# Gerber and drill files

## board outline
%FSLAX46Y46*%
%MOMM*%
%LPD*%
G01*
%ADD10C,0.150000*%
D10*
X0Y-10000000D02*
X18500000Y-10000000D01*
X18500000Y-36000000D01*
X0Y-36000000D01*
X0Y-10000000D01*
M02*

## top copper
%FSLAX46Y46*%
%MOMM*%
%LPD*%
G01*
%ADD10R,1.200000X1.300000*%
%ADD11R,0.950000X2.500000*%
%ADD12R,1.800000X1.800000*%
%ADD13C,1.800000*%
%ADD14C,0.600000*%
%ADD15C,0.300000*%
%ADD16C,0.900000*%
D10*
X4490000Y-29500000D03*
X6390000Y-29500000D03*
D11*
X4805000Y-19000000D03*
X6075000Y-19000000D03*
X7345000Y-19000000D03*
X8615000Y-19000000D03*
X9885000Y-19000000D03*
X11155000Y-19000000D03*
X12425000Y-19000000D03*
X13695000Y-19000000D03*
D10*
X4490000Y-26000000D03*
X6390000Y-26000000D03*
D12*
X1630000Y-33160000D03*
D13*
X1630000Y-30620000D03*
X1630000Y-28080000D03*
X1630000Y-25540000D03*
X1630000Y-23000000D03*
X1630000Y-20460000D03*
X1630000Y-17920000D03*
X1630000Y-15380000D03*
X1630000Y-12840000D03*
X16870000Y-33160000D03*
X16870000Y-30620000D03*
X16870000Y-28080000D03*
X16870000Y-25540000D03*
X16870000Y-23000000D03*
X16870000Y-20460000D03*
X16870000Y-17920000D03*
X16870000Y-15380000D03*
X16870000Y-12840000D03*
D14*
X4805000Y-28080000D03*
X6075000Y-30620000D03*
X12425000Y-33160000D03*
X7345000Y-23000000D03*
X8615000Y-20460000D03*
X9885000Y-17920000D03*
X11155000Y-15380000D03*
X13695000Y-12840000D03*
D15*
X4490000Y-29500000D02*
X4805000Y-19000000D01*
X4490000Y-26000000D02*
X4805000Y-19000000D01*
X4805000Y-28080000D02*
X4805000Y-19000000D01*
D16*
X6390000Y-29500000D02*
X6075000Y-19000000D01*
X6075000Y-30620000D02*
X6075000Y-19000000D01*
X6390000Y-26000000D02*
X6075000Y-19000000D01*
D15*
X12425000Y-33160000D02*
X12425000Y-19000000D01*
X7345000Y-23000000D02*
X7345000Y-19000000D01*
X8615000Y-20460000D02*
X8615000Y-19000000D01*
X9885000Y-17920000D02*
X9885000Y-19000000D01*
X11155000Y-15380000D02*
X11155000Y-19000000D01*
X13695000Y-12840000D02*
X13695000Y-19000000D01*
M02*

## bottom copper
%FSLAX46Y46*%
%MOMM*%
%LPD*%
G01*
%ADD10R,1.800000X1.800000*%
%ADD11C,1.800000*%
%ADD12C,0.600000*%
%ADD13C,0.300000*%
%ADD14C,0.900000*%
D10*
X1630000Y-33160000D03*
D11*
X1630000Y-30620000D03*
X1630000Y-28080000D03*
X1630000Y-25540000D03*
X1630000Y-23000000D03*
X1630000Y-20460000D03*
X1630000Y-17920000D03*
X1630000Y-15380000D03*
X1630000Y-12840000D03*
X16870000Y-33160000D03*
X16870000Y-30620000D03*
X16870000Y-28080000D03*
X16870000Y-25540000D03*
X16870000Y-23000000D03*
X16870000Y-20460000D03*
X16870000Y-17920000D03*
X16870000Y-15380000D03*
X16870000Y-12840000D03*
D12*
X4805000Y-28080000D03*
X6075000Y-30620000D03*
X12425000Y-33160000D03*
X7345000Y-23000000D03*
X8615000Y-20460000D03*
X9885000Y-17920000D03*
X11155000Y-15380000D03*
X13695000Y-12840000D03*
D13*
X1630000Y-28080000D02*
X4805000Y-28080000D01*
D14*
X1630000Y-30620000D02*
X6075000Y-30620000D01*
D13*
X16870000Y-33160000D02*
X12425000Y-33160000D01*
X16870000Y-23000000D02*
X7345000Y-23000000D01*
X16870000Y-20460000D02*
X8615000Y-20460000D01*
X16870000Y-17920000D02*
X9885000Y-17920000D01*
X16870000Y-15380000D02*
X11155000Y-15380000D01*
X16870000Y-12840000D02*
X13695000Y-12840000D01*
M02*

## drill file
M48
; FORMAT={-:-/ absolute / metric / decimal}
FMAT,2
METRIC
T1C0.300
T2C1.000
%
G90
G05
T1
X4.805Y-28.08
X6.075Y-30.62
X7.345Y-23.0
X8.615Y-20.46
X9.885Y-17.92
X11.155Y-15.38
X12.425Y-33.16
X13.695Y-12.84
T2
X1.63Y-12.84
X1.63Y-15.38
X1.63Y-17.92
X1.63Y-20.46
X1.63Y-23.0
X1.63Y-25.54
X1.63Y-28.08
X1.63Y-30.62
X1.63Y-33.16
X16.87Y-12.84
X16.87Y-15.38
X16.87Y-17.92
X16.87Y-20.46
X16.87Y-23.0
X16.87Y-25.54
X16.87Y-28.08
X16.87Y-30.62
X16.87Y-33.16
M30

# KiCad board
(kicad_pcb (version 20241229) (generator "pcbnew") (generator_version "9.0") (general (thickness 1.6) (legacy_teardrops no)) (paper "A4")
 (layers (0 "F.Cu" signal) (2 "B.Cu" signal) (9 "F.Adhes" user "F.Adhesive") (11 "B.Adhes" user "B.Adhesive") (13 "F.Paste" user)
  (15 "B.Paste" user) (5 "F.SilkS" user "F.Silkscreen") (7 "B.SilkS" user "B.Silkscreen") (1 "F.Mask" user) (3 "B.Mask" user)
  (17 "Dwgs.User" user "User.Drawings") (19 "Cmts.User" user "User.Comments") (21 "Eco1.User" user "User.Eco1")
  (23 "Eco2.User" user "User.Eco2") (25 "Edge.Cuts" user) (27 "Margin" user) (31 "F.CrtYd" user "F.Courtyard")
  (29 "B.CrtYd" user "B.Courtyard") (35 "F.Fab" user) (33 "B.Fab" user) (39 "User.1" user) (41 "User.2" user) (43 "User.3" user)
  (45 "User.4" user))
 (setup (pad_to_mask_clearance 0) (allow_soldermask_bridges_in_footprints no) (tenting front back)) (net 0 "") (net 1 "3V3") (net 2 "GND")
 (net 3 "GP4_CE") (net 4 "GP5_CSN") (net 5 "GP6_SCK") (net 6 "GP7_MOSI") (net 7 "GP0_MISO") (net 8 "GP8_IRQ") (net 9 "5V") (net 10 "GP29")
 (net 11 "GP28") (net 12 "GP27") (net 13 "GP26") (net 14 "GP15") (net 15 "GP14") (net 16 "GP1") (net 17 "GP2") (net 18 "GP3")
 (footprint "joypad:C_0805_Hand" (layer "F.Cu") (at 5.44 29.5)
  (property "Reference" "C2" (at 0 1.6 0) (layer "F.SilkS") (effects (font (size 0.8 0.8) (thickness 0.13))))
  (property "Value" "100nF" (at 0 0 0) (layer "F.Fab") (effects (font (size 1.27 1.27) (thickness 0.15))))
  (pad "1" smd rect (at -0.95 0) (size 1.2 1.3) (layers "F.Cu" "F.Mask" "F.Paste") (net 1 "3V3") (thermal_bridge_angle 45))
  (pad "2" smd rect (at 0.95 0) (size 1.2 1.3) (layers "F.Cu" "F.Mask" "F.Paste") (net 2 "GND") (thermal_bridge_angle 45)))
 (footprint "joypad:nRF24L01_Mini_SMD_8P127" (layer "F.Cu") (at 9.25 19)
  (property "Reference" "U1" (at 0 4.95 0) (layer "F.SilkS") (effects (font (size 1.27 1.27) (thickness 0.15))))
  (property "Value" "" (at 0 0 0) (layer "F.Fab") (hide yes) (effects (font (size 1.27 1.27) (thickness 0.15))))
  (pad "1" smd rect (at -4.445 0) (size 0.95 2.5) (layers "F.Cu" "F.Mask" "F.Paste") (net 1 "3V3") (thermal_bridge_angle 45))
  (pad "2" smd rect (at -3.175 0) (size 0.95 2.5) (layers "F.Cu" "F.Mask" "F.Paste") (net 2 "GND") (thermal_bridge_angle 45))
  (pad "3" smd rect (at -1.905 0) (size 0.95 2.5) (layers "F.Cu" "F.Mask" "F.Paste") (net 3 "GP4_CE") (thermal_bridge_angle 45))
  (pad "4" smd rect (at -0.635 0) (size 0.95 2.5) (layers "F.Cu" "F.Mask" "F.Paste") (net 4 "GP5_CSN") (thermal_bridge_angle 45))
  (pad "5" smd rect (at 0.635 0) (size 0.95 2.5) (layers "F.Cu" "F.Mask" "F.Paste") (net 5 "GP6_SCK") (thermal_bridge_angle 45))
  (pad "6" smd rect (at 1.905 0) (size 0.95 2.5) (layers "F.Cu" "F.Mask" "F.Paste") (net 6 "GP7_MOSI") (thermal_bridge_angle 45))
  (pad "7" smd rect (at 3.175 0) (size 0.95 2.5) (layers "F.Cu" "F.Mask" "F.Paste") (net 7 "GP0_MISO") (thermal_bridge_angle 45))
  (pad "8" smd rect (at 4.445 0) (size 0.95 2.5) (layers "F.Cu" "F.Mask" "F.Paste") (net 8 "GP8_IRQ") (thermal_bridge_angle 45))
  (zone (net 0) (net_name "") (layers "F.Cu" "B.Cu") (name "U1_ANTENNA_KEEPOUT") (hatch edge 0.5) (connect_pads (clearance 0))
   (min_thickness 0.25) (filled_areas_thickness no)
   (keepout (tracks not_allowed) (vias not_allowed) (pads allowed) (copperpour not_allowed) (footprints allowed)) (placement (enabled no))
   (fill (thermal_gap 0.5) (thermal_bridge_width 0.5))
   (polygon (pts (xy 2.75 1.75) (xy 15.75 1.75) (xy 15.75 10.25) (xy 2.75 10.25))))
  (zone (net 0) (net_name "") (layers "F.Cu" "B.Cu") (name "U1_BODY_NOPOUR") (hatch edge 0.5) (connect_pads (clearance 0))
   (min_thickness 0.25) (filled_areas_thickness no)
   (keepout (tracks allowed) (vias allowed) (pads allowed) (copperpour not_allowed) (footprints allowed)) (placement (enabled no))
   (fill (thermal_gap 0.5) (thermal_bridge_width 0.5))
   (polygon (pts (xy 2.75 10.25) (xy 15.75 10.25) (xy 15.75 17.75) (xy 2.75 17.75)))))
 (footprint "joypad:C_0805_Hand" (layer "F.Cu") (at 5.44 26)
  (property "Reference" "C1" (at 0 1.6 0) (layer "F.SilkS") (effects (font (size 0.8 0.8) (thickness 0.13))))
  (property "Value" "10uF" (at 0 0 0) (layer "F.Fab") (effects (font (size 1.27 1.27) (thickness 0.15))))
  (pad "1" smd rect (at -0.95 0) (size 1.2 1.3) (layers "F.Cu" "F.Mask" "F.Paste") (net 1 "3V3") (thermal_bridge_angle 45))
  (pad "2" smd rect (at 0.95 0) (size 1.2 1.3) (layers "F.Cu" "F.Mask" "F.Paste") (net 2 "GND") (thermal_bridge_angle 45)))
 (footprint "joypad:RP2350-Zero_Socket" (layer "F.Cu") (at 9.25 23)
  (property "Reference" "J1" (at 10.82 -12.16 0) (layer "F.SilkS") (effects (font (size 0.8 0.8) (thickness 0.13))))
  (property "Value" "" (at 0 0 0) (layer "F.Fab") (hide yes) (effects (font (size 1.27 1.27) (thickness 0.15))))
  (pad "1" thru_hole rect (at -7.62 10.16) (size 1.8 1.8) (drill 1) (layers "*.Cu" "*.Mask") (remove_unused_layers no) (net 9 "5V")
   (thermal_bridge_angle 45))
  (pad "2" thru_hole circle (at -7.62 7.62) (size 1.8 1.8) (drill 1) (layers "*.Cu" "*.Mask") (remove_unused_layers no) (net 2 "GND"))
  (pad "3" thru_hole circle (at -7.62 5.08) (size 1.8 1.8) (drill 1) (layers "*.Cu" "*.Mask") (remove_unused_layers no) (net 1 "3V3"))
  (pad "4" thru_hole circle (at -7.62 2.54) (size 1.8 1.8) (drill 1) (layers "*.Cu" "*.Mask") (remove_unused_layers no) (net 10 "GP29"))
  (pad "5" thru_hole circle (at -7.62 0) (size 1.8 1.8) (drill 1) (layers "*.Cu" "*.Mask") (remove_unused_layers no) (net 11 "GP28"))
  (pad "6" thru_hole circle (at -7.62 -2.54) (size 1.8 1.8) (drill 1) (layers "*.Cu" "*.Mask") (remove_unused_layers no) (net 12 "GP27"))
  (pad "7" thru_hole circle (at -7.62 -5.08) (size 1.8 1.8) (drill 1) (layers "*.Cu" "*.Mask") (remove_unused_layers no) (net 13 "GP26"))
  (pad "8" thru_hole circle (at -7.62 -7.62) (size 1.8 1.8) (drill 1) (layers "*.Cu" "*.Mask") (remove_unused_layers no) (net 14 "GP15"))
  (pad "9" thru_hole circle (at -7.62 -10.16) (size 1.8 1.8) (drill 1) (layers "*.Cu" "*.Mask") (remove_unused_layers no) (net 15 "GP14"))
  (pad "10" thru_hole circle (at 7.62 10.16) (size 1.8 1.8) (drill 1) (layers "*.Cu" "*.Mask") (remove_unused_layers no) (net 7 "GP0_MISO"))
  (pad "11" thru_hole circle (at 7.62 7.62) (size 1.8 1.8) (drill 1) (layers "*.Cu" "*.Mask") (remove_unused_layers no) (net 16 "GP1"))
  (pad "12" thru_hole circle (at 7.62 5.08) (size 1.8 1.8) (drill 1) (layers "*.Cu" "*.Mask") (remove_unused_layers no) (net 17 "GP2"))
  (pad "13" thru_hole circle (at 7.62 2.54) (size 1.8 1.8) (drill 1) (layers "*.Cu" "*.Mask") (remove_unused_layers no) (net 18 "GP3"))
  (pad "14" thru_hole circle (at 7.62 0) (size 1.8 1.8) (drill 1) (layers "*.Cu" "*.Mask") (remove_unused_layers no) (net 3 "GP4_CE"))
  (pad "15" thru_hole circle (at 7.62 -2.54) (size 1.8 1.8) (drill 1) (layers "*.Cu" "*.Mask") (remove_unused_layers no) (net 4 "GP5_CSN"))
  (pad "16" thru_hole circle (at 7.62 -5.08) (size 1.8 1.8) (drill 1) (layers "*.Cu" "*.Mask") (remove_unused_layers no) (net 5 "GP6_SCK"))
  (pad "17" thru_hole circle (at 7.62 -7.62) (size 1.8 1.8) (drill 1) (layers "*.Cu" "*.Mask") (remove_unused_layers no) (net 6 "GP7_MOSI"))
  (pad "18" thru_hole circle (at 7.62 -10.16) (size 1.8 1.8) (drill 1) (layers "*.Cu" "*.Mask") (remove_unused_layers no) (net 8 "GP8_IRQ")))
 (gr_rect (start 0 10) (end 18.5 36) (stroke (width 0.15) (type default)) (fill no) (layer "Edge.Cuts"))
 (segment (start 4.49 29.5) (end 4.805 19) (width 0.3) (layer "F.Cu") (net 1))
 (segment (start 4.49 26) (end 4.805 19) (width 0.3) (layer "F.Cu") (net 1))
 (segment (start 4.805 28.08) (end 4.805 19) (width 0.3) (layer "F.Cu") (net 1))
 (via (at 4.805 28.08) (size 0.6) (drill 0.3) (layers "F.Cu" "B.Cu") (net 1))
 (segment (start 1.63 28.08) (end 4.805 28.08) (width 0.3) (layer "B.Cu") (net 1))
 (segment (start 6.39 29.5) (end 6.075 19) (width 0.9) (layer "F.Cu") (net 2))
 (segment (start 6.075 30.62) (end 6.075 19) (width 0.9) (layer "F.Cu") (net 2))
 (segment (start 6.39 26) (end 6.075 19) (width 0.9) (layer "F.Cu") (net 2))
 (via (at 6.075 30.62) (size 0.6) (drill 0.3) (layers "F.Cu" "B.Cu") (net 2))
 (segment (start 1.63 30.62) (end 6.075 30.62) (width 0.9) (layer "B.Cu") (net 2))
 (segment (start 12.425 33.16) (end 12.425 19) (width 0.3) (layer "F.Cu") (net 7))
 (via (at 12.425 33.16) (size 0.6) (drill 0.3) (layers "F.Cu" "B.Cu") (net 7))
 (segment (start 16.87 33.16) (end 12.425 33.16) (width 0.3) (layer "B.Cu") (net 7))
 (segment (start 7.345 23) (end 7.345 19) (width 0.3) (layer "F.Cu") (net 3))
 (via (at 7.345 23) (size 0.6) (drill 0.3) (layers "F.Cu" "B.Cu") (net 3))
 (segment (start 16.87 23) (end 7.345 23) (width 0.3) (layer "B.Cu") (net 3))
 (segment (start 8.615 20.46) (end 8.615 19) (width 0.3) (layer "F.Cu") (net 4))
 (via (at 8.615 20.46) (size 0.6) (drill 0.3) (layers "F.Cu" "B.Cu") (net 4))
 (segment (start 16.87 20.46) (end 8.615 20.46) (width 0.3) (layer "B.Cu") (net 4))
 (segment (start 9.885 17.92) (end 9.885 19) (width 0.3) (layer "F.Cu") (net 5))
 (via (at 9.885 17.92) (size 0.6) (drill 0.3) (layers "F.Cu" "B.Cu") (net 5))
 (segment (start 16.87 17.92) (end 9.885 17.92) (width 0.3) (layer "B.Cu") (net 5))
 (segment (start 11.155 15.38) (end 11.155 19) (width 0.3) (layer "F.Cu") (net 6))
 (via (at 11.155 15.38) (size 0.6) (drill 0.3) (layers "F.Cu" "B.Cu") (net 6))
 (segment (start 16.87 15.38) (end 11.155 15.38) (width 0.3) (layer "B.Cu") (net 6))
 (segment (start 13.695 12.84) (end 13.695 19) (width 0.3) (layer "F.Cu") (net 8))
 (via (at 13.695 12.84) (size 0.6) (drill 0.3) (layers "F.Cu" "B.Cu") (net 8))
 (segment (start 16.87 12.84) (end 13.695 12.84) (width 0.3) (layer "B.Cu") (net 8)))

